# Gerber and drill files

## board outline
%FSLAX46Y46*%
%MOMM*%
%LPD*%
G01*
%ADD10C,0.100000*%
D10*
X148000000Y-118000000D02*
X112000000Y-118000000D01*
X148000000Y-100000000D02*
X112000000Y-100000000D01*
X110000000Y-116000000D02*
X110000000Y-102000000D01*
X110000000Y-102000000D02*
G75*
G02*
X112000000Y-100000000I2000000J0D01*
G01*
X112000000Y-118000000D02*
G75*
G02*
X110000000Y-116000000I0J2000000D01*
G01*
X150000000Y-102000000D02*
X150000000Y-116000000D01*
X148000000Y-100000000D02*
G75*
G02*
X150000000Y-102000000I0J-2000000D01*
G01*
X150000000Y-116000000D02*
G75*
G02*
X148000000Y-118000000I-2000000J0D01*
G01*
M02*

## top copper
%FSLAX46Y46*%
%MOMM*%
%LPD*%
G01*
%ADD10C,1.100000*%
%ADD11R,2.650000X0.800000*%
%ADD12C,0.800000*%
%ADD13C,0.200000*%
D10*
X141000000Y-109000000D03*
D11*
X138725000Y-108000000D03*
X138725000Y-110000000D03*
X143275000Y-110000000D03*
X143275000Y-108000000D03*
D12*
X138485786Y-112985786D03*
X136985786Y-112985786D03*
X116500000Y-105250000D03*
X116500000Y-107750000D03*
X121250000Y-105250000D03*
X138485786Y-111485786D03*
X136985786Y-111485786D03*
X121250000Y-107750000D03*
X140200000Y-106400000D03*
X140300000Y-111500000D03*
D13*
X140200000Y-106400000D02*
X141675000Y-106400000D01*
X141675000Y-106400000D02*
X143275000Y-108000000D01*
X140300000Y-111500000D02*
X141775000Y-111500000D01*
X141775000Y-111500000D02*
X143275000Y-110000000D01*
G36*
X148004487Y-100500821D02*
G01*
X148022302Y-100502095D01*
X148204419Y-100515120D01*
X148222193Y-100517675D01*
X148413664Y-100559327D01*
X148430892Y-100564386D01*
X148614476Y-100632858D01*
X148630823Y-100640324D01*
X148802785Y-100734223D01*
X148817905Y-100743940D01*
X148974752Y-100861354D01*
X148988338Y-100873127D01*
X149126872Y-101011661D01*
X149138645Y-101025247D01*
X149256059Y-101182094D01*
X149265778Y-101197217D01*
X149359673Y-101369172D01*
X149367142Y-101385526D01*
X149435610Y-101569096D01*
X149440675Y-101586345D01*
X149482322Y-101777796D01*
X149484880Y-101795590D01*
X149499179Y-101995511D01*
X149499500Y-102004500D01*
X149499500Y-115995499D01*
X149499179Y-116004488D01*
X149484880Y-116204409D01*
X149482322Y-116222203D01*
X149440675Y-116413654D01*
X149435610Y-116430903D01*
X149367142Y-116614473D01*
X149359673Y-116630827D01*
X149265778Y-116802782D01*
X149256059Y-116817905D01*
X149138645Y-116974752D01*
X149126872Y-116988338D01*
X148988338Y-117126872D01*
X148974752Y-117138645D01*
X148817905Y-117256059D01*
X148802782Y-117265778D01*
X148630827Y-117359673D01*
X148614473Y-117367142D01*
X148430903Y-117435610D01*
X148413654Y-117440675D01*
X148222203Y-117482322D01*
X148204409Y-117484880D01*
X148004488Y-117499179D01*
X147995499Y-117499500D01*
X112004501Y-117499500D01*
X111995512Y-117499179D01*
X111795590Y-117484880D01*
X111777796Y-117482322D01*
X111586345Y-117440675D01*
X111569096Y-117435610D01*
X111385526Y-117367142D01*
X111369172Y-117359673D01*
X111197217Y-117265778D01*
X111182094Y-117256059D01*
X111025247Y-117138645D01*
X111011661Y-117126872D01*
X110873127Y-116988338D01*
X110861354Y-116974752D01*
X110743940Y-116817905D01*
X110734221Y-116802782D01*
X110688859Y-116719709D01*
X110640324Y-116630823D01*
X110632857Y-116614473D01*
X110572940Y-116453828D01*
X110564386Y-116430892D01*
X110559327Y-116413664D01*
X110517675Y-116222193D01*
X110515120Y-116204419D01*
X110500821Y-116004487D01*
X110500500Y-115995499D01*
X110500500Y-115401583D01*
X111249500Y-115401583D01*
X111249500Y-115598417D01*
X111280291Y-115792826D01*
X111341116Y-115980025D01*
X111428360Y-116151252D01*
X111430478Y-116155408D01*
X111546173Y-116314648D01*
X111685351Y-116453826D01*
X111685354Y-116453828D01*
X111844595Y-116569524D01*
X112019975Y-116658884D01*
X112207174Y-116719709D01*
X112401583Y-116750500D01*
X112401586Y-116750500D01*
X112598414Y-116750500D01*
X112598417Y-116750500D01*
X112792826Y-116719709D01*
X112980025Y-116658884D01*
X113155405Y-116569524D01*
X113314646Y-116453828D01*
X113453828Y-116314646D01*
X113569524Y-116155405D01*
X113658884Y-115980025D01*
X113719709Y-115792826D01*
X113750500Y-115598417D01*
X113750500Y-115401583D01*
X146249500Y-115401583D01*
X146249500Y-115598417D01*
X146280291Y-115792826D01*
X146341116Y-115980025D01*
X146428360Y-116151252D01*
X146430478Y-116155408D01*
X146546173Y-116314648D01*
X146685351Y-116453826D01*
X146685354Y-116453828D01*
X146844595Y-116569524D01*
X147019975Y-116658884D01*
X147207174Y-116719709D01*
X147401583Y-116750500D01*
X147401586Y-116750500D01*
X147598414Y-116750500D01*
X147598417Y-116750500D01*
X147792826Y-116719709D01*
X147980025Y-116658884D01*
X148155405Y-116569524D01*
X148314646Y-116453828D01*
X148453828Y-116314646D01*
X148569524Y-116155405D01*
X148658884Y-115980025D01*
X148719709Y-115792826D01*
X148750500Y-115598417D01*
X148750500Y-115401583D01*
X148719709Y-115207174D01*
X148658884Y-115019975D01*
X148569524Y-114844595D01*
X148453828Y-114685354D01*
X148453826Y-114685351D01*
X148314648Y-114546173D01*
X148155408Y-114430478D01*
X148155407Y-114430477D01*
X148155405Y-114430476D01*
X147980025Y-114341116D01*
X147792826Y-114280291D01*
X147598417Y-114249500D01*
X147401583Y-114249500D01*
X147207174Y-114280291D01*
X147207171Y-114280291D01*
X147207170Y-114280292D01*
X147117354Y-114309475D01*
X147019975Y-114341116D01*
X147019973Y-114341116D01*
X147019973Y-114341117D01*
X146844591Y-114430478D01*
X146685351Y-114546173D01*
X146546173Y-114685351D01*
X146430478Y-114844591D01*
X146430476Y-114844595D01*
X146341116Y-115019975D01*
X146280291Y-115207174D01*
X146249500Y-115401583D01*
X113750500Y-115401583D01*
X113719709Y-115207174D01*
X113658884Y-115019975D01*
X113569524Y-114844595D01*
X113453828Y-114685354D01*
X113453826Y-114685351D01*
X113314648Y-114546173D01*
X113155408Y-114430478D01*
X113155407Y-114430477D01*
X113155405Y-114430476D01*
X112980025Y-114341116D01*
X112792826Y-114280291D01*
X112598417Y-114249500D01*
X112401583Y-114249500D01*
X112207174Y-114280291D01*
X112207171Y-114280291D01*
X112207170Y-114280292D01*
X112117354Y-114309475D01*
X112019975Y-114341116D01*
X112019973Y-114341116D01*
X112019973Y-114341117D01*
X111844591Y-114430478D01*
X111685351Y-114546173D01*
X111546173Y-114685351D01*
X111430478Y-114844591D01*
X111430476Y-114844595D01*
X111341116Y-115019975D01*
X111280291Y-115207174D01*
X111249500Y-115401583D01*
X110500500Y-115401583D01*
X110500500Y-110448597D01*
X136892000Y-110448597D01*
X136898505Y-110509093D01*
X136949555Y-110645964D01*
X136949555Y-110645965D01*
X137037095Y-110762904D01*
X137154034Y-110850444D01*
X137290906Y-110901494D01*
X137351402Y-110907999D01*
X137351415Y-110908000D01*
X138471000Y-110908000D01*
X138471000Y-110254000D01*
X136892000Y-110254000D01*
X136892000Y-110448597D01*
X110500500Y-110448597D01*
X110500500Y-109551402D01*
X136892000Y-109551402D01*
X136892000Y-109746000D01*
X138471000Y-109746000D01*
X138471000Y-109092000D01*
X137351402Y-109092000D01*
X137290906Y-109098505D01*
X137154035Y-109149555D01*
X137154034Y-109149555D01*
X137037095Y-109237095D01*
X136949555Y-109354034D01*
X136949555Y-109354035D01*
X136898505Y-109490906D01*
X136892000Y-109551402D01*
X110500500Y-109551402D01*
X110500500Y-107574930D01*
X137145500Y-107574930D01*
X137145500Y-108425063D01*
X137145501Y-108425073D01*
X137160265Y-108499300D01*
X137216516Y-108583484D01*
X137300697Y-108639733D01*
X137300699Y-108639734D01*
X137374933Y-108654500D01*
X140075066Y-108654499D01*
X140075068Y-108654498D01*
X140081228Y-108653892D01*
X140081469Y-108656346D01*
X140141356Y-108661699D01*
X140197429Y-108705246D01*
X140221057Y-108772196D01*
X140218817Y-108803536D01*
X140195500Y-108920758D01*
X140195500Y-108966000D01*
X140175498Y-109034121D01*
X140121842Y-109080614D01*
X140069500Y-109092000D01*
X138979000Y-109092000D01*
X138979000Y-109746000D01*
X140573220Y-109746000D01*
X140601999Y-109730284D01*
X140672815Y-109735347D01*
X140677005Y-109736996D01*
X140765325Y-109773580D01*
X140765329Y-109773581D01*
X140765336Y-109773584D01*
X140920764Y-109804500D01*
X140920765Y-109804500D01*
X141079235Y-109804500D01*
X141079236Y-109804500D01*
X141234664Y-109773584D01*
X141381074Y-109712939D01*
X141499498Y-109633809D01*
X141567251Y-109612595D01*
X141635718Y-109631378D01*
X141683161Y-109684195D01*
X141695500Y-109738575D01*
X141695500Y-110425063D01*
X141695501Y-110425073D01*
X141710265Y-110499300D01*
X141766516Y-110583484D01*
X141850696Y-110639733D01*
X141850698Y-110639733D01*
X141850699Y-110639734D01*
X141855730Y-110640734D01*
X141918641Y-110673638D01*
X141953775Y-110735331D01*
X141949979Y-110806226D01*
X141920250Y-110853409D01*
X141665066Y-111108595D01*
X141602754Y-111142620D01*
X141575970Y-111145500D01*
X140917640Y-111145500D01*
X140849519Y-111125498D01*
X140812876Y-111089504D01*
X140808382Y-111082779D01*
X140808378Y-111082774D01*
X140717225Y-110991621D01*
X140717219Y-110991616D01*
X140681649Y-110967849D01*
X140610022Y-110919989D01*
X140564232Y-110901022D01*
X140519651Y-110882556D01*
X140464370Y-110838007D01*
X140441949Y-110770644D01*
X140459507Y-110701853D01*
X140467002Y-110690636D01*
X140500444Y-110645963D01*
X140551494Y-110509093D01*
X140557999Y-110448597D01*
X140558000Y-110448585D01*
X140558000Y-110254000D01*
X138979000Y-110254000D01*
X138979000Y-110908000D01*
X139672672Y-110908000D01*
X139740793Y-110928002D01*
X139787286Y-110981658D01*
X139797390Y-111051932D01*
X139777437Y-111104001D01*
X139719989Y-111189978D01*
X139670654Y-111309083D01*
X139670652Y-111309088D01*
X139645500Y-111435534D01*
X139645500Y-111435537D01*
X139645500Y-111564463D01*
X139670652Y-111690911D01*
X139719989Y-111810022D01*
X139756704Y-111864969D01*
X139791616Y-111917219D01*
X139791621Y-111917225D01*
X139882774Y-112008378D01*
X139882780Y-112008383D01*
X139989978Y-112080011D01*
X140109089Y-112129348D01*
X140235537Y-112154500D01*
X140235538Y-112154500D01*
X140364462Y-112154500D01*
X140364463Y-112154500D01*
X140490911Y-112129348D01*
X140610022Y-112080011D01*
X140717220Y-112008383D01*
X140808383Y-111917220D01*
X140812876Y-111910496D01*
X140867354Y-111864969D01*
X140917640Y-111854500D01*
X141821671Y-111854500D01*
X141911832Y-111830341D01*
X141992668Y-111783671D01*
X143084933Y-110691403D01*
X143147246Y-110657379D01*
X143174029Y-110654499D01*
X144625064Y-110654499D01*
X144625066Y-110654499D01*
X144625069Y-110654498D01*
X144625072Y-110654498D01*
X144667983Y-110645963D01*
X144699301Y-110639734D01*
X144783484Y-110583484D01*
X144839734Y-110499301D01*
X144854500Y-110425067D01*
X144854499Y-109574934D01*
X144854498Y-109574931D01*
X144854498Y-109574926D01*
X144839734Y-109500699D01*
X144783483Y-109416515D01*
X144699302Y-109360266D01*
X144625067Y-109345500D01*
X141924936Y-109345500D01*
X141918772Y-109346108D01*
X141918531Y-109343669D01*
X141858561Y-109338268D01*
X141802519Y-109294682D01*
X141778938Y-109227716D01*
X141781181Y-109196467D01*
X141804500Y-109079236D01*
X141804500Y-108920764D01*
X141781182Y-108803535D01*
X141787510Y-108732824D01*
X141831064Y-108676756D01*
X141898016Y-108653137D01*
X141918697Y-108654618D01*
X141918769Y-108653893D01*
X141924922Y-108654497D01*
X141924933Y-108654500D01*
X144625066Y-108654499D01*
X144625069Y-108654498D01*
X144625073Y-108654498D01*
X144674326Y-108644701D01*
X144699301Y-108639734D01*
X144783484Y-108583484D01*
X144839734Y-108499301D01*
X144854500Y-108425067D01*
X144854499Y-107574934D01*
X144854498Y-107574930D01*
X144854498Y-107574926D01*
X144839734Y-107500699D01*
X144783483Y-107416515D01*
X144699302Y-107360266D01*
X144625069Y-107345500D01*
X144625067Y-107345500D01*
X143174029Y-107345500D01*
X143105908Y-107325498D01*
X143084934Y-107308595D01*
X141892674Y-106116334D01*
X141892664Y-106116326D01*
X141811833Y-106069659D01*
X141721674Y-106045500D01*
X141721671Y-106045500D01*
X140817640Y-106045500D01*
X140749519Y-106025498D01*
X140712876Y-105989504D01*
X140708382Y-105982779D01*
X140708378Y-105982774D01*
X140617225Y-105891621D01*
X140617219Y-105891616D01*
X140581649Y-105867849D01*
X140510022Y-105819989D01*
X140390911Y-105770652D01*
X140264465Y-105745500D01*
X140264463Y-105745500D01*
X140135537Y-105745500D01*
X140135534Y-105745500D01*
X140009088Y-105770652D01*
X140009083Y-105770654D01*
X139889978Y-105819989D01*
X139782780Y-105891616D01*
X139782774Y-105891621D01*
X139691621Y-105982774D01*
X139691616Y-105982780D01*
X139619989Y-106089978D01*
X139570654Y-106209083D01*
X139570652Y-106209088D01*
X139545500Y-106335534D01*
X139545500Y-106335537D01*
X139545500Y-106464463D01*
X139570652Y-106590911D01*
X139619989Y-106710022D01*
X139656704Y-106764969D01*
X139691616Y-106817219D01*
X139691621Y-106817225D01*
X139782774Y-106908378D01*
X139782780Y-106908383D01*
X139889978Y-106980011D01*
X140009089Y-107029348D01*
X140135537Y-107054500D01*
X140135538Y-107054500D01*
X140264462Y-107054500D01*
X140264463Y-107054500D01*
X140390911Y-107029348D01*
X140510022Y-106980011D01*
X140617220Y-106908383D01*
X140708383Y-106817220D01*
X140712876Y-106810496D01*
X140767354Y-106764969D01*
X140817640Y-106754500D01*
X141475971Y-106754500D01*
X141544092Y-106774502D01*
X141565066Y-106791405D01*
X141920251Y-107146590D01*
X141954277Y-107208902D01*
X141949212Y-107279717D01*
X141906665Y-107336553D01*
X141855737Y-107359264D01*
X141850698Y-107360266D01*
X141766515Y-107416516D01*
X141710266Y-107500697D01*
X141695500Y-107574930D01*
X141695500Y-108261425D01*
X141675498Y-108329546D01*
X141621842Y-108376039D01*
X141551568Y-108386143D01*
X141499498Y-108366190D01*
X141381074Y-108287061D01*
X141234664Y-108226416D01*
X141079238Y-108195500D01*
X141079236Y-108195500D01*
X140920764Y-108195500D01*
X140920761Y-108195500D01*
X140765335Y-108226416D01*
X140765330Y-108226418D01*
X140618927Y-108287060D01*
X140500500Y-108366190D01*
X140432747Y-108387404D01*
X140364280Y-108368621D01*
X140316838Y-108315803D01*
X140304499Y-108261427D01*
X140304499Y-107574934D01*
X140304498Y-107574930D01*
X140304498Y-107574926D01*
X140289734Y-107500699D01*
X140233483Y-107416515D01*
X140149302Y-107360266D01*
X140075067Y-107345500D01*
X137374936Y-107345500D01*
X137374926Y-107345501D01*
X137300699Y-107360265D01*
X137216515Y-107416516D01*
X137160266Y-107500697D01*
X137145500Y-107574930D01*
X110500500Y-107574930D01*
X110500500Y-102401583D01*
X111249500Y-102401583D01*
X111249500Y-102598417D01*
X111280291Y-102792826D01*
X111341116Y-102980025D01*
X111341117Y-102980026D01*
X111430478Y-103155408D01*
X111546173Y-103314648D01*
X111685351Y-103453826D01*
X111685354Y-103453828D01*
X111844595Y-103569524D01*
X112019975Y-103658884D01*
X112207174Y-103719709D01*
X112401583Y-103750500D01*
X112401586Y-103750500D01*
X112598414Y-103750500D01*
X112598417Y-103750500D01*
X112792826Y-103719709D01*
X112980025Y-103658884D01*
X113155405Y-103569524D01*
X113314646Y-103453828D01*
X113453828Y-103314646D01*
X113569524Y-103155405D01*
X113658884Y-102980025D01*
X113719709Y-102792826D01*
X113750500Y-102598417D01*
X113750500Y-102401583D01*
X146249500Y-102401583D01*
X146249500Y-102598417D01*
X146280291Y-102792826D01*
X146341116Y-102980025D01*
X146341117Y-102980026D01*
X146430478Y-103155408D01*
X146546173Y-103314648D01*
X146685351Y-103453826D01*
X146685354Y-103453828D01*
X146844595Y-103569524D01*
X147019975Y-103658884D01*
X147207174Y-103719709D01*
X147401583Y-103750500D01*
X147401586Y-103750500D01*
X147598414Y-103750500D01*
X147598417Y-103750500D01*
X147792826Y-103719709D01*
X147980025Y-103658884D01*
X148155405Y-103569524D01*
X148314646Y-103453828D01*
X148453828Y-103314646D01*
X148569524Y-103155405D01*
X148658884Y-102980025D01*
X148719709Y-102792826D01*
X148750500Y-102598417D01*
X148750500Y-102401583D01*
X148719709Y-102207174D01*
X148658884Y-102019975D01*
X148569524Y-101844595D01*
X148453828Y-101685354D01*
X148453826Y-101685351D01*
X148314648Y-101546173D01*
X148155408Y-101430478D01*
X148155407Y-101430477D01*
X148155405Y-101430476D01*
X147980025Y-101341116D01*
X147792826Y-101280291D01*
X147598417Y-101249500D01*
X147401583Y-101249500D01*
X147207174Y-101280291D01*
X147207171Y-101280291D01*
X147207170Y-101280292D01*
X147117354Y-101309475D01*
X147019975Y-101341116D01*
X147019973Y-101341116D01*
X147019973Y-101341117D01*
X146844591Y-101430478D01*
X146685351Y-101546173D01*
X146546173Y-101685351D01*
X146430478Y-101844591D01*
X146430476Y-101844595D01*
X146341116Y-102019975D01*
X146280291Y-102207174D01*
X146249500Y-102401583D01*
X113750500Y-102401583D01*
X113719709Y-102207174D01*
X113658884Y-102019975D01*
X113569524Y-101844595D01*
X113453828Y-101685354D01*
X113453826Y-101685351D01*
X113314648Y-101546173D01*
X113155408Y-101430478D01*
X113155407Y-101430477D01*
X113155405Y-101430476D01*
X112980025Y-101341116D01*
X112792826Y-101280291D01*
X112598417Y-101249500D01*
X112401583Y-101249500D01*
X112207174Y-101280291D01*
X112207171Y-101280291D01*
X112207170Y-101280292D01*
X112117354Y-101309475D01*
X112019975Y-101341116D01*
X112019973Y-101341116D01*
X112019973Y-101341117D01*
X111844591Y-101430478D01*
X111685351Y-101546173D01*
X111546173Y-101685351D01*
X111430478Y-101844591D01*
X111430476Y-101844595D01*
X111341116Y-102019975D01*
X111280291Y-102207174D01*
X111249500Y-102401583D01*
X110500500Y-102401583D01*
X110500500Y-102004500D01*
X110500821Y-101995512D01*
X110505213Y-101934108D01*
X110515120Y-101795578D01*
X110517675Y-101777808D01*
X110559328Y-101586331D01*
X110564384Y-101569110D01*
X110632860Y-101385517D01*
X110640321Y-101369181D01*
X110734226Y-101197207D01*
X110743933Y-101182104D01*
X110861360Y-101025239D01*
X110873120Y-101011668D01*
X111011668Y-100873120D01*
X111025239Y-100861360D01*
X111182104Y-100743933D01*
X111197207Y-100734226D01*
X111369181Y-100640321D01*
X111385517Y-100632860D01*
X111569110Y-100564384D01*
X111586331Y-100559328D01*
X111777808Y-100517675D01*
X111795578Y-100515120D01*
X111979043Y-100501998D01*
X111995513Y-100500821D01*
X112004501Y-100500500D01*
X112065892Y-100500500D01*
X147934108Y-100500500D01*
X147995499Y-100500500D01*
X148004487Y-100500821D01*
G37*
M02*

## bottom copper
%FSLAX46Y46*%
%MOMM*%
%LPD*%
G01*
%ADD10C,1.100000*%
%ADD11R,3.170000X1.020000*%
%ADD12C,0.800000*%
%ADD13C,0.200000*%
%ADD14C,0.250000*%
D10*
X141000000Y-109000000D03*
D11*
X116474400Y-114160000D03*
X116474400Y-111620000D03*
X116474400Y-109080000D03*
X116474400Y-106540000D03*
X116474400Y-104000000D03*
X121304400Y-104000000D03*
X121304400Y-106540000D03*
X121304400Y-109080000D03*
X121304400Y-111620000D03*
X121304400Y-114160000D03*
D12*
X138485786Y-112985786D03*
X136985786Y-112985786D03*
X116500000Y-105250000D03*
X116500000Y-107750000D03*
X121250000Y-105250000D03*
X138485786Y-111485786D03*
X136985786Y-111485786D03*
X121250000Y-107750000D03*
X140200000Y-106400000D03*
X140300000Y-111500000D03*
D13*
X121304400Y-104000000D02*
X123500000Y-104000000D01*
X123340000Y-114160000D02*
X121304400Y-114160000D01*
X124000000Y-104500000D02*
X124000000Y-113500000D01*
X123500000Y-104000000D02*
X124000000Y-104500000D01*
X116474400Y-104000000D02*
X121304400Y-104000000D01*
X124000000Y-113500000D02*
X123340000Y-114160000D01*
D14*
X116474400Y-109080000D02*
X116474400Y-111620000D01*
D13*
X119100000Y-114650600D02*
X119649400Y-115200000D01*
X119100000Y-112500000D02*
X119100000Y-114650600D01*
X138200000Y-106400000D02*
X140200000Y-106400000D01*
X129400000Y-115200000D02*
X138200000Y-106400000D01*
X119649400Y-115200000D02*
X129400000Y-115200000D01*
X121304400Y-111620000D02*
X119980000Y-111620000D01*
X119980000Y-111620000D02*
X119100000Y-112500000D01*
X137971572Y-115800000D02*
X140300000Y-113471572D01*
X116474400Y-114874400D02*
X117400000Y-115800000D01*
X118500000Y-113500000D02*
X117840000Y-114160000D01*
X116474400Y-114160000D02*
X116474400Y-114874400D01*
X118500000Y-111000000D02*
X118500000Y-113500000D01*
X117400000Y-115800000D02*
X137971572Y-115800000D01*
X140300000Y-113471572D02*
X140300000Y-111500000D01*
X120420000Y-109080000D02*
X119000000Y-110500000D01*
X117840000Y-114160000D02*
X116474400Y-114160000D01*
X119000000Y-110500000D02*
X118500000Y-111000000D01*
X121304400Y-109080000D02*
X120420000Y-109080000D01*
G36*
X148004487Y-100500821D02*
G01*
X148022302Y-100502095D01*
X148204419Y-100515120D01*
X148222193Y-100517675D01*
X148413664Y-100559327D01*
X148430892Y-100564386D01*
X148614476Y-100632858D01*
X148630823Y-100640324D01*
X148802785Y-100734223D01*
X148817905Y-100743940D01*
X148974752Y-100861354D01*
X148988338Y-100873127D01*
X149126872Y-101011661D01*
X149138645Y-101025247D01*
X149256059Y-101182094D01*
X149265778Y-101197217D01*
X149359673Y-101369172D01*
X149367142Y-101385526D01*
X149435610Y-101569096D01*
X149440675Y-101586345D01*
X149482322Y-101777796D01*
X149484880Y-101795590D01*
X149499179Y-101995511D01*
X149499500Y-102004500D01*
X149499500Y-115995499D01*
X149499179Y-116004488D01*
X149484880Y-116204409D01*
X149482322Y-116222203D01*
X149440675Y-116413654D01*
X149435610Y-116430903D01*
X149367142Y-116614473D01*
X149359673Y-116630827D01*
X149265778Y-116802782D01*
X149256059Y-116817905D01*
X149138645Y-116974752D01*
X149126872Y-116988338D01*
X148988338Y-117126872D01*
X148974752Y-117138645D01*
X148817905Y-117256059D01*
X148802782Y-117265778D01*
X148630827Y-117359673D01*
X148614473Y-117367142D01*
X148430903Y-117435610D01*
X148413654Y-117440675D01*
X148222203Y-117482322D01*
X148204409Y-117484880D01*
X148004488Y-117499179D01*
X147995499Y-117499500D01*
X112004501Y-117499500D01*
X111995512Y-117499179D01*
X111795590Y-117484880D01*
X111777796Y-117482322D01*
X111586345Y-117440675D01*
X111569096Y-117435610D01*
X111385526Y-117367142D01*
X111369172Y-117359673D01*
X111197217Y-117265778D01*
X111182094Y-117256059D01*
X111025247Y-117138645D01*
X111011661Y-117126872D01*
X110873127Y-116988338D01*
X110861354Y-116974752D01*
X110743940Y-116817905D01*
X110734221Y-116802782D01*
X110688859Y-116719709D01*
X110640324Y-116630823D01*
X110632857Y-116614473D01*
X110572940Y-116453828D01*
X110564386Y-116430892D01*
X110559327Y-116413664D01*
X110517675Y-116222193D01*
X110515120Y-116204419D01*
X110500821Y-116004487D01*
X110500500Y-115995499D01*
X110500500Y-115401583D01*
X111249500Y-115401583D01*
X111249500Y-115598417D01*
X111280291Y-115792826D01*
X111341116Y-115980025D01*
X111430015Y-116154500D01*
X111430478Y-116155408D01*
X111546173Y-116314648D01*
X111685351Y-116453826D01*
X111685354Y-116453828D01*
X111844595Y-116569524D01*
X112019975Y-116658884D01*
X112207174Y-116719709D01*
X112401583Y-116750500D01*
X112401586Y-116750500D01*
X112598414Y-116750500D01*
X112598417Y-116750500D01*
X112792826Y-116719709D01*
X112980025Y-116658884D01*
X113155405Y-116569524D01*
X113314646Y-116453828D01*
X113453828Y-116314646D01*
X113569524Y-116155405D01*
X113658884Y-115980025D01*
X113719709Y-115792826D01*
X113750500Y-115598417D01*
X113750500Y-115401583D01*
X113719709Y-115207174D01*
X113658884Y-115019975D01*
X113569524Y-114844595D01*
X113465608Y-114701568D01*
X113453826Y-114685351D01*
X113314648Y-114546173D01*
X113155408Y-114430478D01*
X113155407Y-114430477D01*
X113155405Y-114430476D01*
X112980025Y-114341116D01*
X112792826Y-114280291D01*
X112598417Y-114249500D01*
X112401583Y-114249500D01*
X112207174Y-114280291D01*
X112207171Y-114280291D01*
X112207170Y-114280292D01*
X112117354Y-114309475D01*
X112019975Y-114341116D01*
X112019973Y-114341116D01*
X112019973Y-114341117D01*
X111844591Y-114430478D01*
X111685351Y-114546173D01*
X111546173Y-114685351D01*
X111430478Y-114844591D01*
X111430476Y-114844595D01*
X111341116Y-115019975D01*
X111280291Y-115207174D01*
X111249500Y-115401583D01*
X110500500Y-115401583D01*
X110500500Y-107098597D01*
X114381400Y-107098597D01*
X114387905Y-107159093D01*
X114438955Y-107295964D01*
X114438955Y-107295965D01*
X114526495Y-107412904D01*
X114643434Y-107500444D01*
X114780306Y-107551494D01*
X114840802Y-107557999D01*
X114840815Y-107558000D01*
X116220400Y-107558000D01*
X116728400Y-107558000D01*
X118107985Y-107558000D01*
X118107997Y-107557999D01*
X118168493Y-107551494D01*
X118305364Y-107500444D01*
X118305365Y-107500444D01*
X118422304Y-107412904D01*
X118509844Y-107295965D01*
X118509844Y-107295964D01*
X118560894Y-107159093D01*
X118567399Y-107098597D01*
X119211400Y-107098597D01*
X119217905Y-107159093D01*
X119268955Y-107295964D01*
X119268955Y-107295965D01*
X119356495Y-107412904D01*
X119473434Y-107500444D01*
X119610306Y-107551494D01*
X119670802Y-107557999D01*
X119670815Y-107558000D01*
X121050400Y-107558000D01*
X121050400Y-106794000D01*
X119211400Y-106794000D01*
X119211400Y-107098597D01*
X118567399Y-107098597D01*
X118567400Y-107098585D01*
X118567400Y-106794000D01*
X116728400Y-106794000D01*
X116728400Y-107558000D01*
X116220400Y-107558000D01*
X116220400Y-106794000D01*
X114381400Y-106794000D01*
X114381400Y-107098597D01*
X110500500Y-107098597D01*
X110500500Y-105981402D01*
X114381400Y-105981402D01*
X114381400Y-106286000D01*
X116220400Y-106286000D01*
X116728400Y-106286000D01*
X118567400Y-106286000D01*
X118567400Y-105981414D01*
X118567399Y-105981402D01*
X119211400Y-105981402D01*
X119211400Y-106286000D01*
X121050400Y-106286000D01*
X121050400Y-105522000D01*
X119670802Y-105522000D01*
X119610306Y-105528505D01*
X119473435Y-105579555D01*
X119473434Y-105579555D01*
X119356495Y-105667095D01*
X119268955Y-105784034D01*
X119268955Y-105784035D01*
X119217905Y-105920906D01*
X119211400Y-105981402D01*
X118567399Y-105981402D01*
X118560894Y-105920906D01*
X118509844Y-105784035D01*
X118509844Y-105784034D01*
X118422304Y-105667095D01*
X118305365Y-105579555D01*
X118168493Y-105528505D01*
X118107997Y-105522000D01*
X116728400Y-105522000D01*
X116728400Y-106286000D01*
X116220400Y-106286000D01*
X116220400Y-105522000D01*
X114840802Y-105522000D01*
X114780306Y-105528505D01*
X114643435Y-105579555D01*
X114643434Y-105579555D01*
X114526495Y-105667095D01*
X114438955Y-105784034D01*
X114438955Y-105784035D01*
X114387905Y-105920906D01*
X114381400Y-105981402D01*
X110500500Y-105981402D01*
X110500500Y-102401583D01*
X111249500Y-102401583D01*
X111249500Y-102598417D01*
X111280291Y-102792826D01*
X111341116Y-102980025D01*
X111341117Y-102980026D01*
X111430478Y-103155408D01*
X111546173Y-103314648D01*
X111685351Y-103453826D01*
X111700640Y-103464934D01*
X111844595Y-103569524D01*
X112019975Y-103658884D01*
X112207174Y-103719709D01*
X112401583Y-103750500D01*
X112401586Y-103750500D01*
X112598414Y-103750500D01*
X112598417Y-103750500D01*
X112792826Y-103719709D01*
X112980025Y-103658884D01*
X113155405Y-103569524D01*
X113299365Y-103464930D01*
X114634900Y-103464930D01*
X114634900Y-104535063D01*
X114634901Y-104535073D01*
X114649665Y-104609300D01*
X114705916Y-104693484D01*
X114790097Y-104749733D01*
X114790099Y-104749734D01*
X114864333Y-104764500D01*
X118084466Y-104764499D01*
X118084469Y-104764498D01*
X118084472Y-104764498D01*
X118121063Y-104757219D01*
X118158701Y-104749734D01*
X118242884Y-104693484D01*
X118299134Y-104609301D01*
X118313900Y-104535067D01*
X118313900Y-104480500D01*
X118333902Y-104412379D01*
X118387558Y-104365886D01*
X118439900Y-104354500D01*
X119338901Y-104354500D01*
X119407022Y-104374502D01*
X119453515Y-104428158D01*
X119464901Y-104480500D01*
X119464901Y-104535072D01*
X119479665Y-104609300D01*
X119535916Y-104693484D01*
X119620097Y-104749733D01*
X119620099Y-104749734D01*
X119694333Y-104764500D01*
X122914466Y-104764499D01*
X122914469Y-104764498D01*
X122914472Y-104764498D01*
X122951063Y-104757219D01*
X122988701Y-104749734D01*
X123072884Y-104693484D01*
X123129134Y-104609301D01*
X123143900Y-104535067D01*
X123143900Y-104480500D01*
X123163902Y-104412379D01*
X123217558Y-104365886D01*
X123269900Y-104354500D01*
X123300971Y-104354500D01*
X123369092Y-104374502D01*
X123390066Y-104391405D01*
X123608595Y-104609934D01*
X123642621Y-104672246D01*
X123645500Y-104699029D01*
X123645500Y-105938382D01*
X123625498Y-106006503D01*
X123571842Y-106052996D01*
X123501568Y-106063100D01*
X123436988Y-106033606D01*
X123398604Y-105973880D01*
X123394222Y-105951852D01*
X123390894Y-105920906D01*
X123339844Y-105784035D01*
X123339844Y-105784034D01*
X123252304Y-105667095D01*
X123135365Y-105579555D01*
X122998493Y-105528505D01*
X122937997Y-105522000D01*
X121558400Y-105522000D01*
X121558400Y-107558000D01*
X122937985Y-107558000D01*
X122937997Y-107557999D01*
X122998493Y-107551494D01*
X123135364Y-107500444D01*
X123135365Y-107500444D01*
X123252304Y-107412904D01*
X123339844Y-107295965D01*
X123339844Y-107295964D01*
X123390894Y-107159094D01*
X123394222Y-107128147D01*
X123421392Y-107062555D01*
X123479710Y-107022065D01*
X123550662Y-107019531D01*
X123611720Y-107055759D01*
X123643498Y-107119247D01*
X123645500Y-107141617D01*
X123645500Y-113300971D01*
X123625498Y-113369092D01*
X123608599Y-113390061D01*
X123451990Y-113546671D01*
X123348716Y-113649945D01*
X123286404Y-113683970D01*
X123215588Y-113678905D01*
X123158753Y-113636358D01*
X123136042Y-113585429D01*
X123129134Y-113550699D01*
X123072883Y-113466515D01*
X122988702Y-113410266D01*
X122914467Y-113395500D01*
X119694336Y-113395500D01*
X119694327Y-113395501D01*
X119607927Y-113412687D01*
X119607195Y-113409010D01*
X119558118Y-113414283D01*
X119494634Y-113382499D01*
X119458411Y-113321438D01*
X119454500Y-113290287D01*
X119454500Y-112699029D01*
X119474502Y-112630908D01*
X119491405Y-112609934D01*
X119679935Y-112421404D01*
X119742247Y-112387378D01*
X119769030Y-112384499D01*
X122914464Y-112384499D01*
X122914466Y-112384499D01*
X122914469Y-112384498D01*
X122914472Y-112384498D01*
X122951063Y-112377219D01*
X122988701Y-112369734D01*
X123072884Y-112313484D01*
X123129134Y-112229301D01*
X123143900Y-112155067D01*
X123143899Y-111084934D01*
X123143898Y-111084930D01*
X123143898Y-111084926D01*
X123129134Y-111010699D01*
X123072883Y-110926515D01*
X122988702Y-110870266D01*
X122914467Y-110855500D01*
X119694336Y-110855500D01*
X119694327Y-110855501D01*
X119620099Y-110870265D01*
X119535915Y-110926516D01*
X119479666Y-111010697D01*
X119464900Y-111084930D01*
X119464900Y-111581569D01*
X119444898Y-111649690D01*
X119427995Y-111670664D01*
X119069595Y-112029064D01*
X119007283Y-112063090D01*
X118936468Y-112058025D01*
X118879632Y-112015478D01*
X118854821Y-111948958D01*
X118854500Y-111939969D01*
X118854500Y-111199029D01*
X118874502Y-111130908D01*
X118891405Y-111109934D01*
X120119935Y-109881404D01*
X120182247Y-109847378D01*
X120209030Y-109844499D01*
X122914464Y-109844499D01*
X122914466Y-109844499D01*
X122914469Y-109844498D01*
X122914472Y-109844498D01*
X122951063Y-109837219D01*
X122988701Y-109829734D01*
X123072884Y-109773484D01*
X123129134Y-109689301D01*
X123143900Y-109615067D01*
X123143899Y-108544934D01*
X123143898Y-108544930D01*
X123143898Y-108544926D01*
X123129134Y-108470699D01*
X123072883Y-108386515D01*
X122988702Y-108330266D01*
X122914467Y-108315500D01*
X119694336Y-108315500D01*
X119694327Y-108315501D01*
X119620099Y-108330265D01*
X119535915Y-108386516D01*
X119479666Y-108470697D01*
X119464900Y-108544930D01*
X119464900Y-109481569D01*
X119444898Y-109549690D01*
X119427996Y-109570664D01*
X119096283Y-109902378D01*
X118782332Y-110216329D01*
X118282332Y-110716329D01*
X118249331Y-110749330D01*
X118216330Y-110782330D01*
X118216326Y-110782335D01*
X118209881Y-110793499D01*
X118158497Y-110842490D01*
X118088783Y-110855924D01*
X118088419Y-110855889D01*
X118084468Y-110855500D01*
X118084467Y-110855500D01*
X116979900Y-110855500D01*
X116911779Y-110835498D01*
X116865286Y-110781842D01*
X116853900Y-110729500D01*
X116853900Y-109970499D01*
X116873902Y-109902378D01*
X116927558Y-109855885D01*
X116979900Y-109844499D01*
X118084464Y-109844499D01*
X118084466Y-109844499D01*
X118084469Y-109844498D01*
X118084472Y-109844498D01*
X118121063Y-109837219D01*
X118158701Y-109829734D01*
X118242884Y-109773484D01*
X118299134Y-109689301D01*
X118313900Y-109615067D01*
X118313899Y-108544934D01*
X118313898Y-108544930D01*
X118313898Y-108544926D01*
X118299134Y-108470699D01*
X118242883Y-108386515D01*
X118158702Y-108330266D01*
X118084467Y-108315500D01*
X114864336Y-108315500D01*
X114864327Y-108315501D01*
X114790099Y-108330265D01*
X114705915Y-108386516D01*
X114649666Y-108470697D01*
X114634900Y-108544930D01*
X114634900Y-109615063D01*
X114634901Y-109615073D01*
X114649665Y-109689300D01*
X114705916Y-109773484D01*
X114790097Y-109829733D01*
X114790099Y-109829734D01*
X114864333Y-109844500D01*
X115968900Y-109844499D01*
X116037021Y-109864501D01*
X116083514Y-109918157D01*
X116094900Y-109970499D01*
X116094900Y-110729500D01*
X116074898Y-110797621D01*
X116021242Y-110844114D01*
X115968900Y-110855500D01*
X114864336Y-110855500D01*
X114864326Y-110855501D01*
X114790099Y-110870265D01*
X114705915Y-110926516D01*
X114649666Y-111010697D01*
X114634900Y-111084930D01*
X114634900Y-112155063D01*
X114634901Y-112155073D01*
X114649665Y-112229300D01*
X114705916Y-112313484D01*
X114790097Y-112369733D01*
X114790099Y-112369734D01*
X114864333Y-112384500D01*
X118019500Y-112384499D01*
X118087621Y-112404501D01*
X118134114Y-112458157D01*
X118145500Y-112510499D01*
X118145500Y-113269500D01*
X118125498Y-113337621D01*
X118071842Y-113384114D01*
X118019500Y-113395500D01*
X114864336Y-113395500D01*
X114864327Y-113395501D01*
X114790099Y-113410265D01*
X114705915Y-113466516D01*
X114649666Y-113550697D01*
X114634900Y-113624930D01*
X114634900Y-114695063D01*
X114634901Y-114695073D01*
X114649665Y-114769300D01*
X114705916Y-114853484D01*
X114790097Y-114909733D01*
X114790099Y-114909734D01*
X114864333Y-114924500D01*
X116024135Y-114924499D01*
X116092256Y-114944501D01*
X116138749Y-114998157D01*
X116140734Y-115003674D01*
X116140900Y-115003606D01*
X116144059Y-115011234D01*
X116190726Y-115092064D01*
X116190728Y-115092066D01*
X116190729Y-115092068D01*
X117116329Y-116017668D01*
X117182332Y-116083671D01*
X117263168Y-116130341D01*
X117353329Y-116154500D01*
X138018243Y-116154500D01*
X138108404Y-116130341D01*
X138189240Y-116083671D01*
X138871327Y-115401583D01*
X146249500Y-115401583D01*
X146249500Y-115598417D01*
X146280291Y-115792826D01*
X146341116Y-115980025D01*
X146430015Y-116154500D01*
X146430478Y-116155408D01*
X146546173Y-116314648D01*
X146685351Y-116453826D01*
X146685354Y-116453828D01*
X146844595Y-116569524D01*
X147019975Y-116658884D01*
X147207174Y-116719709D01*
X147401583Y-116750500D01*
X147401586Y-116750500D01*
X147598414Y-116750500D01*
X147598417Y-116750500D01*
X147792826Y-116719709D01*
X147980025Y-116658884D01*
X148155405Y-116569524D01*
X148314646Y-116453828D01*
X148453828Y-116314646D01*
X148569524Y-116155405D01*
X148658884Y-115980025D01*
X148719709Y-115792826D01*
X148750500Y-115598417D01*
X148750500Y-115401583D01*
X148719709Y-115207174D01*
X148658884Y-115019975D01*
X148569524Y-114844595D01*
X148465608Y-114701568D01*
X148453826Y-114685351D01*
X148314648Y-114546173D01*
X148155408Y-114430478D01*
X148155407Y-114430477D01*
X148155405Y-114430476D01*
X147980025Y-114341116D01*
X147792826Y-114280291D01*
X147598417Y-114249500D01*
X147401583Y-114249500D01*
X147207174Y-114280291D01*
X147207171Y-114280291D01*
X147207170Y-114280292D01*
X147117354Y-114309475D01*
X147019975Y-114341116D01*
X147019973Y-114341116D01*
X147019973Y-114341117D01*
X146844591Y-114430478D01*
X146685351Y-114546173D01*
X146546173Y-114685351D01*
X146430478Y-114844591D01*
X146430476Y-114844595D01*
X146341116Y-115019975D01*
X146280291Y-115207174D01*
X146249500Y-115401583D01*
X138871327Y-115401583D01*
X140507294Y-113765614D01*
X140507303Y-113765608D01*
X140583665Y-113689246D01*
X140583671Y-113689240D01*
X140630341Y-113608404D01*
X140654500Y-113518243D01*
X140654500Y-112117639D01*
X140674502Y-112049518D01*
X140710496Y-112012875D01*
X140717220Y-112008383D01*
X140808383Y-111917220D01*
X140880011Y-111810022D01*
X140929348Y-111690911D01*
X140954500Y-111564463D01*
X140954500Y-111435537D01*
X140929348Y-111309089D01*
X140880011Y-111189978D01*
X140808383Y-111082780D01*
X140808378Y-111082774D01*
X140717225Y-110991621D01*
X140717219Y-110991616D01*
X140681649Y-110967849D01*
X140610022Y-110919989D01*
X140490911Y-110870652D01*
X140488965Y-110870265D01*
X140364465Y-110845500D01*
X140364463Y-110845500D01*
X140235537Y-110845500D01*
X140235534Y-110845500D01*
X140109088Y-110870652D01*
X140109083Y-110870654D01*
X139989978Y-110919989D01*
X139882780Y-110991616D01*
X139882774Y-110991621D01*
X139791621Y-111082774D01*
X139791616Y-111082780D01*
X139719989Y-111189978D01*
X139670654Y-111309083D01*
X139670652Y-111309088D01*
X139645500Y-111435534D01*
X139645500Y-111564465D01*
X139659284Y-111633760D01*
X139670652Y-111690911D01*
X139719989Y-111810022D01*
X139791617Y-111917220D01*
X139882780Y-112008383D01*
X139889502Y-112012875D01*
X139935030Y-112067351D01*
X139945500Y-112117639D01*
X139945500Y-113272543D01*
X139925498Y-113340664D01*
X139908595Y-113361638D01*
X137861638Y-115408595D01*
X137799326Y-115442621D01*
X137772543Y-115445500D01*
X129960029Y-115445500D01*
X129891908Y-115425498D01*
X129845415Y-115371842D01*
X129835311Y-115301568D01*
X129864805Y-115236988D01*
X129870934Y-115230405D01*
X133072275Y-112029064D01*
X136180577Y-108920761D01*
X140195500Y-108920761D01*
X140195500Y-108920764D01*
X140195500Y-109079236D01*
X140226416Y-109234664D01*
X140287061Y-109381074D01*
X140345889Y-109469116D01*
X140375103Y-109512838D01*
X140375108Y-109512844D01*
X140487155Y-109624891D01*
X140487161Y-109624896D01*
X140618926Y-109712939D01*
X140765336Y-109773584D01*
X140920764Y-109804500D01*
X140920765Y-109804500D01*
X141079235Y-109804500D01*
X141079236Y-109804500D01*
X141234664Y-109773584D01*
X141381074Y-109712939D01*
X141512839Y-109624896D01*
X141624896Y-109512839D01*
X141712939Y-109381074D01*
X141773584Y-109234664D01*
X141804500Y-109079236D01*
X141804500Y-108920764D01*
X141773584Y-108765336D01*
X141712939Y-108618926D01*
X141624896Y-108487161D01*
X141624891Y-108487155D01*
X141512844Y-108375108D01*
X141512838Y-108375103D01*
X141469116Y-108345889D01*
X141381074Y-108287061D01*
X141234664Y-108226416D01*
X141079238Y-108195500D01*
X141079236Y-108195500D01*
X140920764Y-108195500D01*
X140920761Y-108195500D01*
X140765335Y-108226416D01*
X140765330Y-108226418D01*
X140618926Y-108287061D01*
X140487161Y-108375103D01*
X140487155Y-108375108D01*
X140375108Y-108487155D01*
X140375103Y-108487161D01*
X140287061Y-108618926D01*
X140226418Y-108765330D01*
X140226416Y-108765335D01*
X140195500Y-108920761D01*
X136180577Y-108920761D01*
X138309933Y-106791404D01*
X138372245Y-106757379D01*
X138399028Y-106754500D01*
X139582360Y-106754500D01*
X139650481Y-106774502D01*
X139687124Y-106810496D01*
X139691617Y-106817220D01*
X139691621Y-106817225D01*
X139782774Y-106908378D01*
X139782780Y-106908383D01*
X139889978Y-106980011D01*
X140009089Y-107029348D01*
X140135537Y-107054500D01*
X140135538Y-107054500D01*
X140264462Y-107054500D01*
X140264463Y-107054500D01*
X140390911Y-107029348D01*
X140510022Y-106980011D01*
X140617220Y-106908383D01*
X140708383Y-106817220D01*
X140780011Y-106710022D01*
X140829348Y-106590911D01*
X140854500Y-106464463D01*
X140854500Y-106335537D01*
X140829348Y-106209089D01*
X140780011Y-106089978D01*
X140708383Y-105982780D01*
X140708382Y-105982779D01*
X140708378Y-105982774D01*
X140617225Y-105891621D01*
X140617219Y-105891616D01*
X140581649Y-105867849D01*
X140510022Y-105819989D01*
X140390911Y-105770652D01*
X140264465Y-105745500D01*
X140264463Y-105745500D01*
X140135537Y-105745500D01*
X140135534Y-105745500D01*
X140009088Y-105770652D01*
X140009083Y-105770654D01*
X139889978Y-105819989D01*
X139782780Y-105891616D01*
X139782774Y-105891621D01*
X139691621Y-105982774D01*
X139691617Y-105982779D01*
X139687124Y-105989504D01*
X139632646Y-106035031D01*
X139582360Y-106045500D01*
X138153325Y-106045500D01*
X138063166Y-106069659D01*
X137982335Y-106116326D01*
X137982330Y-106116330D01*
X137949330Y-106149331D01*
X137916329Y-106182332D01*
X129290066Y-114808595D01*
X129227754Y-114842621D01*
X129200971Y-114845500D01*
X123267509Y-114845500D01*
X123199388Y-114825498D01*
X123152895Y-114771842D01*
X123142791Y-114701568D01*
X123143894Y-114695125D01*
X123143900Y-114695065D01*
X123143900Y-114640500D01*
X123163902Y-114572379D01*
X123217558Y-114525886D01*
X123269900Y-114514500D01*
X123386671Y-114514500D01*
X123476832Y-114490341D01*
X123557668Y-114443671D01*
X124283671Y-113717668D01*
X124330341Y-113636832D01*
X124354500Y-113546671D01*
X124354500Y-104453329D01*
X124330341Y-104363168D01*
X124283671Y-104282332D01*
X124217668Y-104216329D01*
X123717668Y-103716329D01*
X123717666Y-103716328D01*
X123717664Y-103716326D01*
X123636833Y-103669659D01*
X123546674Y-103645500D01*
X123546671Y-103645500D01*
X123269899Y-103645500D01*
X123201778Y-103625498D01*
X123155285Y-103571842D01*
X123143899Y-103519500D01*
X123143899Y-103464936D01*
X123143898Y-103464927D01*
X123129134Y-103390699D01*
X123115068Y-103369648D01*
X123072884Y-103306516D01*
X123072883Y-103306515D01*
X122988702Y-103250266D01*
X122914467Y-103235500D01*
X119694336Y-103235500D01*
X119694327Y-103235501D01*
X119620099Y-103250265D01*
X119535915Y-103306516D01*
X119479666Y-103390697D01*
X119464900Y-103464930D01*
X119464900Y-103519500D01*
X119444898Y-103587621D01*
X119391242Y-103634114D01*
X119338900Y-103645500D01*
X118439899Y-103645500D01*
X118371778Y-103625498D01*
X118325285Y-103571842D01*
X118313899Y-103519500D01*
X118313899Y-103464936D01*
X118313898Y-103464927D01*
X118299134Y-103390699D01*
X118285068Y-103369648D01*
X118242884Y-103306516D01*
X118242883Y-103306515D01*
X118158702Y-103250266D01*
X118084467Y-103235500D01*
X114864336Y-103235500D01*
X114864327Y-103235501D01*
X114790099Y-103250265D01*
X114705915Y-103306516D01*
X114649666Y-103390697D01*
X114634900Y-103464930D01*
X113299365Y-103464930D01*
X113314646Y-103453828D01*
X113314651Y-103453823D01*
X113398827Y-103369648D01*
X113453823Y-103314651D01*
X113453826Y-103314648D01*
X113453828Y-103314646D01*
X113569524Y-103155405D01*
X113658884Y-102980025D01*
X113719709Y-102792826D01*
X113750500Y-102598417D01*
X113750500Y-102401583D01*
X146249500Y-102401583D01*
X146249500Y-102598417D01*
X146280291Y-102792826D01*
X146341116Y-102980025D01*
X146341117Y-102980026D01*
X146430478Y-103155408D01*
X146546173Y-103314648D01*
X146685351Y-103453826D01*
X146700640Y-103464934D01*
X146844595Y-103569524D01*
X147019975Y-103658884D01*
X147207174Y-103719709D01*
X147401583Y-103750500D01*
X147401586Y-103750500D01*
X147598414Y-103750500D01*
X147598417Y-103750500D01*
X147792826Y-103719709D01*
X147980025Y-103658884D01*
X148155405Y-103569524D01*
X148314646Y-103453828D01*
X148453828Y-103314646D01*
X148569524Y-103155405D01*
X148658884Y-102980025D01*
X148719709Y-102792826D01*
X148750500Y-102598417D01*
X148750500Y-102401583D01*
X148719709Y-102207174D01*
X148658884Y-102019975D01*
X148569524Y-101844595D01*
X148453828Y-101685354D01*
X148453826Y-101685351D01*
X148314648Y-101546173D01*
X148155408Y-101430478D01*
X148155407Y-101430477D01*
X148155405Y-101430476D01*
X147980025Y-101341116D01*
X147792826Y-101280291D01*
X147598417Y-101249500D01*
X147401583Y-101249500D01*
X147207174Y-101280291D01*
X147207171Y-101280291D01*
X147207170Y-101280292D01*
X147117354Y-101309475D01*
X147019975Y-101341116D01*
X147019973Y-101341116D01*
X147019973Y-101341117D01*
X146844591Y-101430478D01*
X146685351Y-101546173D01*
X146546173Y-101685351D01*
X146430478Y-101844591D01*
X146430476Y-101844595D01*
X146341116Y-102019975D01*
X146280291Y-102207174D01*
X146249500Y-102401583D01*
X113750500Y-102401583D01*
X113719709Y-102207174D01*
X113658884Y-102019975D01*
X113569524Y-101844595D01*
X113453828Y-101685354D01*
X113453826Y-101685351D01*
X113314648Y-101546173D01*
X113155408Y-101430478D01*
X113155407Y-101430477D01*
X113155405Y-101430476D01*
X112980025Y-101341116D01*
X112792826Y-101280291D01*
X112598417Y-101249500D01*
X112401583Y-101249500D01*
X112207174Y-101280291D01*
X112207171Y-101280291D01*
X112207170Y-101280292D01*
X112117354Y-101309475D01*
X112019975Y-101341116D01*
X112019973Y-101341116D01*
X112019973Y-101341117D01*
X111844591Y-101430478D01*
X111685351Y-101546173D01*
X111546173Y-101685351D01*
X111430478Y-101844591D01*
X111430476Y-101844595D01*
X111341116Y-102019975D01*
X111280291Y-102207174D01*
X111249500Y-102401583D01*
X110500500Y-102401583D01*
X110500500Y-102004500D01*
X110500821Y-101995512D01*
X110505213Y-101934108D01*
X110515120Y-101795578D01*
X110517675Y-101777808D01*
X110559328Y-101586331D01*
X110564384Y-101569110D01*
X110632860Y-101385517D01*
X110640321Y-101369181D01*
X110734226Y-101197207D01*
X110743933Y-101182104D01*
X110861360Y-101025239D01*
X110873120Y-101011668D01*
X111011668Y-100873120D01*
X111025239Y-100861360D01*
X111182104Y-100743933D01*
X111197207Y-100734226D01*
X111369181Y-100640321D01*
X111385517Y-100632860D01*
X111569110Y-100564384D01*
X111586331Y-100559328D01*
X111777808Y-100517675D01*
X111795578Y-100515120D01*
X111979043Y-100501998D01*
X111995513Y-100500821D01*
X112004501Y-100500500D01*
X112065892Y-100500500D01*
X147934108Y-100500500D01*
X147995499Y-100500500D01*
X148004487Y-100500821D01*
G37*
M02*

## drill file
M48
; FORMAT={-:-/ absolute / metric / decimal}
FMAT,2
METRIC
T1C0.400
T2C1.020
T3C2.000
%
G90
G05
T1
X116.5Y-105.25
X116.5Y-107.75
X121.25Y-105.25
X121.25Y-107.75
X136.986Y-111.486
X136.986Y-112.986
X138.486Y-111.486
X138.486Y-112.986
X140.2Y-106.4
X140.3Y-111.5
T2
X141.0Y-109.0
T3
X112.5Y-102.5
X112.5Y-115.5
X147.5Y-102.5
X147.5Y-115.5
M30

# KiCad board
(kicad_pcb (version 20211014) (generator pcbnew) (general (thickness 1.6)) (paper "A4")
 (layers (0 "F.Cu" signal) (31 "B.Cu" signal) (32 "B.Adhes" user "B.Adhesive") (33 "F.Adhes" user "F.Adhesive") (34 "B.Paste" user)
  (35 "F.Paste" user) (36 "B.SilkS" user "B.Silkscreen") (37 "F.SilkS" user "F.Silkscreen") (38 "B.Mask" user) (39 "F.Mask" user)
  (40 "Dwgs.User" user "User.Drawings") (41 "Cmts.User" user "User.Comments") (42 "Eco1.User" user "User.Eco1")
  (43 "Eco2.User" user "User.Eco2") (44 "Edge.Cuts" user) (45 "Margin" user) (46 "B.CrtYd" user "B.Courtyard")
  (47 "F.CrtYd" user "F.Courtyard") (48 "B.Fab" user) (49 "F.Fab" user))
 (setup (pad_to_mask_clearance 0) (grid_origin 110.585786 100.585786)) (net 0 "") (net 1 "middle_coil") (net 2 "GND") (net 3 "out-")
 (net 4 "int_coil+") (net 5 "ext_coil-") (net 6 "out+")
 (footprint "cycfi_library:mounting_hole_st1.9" (layer "F.Cu") (at 147.5 115.5 180)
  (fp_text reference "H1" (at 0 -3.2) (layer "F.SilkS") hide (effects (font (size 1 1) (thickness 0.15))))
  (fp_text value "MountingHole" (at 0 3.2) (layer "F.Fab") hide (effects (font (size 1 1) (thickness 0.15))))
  (pad "" np_thru_hole circle locked (at 0 0 180) (size 2 2) (drill 2) (layers *.Cu *.Mask)))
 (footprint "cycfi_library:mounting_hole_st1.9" (layer "F.Cu") (at 147.5 102.5 180)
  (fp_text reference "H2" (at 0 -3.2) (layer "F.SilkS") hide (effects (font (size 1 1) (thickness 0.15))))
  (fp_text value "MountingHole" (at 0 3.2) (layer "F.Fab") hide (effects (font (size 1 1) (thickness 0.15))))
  (pad "" np_thru_hole circle locked (at 0 0 180) (size 2 2) (drill 2) (layers *.Cu *.Mask)))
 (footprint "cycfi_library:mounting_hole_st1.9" (layer "F.Cu") (at 112.5 115.5 180)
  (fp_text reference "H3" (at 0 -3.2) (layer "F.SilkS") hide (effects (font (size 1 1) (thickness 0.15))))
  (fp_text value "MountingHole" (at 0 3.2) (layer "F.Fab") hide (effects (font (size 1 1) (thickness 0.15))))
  (pad "" np_thru_hole circle locked (at 0 0 180) (size 2 2) (drill 2) (layers *.Cu *.Mask)))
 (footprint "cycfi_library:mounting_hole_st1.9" (layer "F.Cu") (at 112.5 102.5 180)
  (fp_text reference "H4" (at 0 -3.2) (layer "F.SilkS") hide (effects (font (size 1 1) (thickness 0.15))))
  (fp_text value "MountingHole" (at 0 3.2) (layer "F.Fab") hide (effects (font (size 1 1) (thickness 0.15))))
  (pad "" np_thru_hole circle locked (at 0 0 180) (size 2 2) (drill 2) (layers *.Cu *.Mask)))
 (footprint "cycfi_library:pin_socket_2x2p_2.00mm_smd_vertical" (layer "F.Cu") (at 141 109)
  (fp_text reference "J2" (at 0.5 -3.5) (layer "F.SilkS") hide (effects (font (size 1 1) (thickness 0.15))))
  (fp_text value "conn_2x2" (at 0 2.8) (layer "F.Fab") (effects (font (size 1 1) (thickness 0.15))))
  (pad "" np_thru_hole circle (at 0 0) (size 1.1 1.1) (drill 1.02) (layers F&B.Cu *.Mask))
  (pad "1" smd rect (at -2.275 -1) (size 2.65 0.8) (layers "F.Cu" "F.Paste" "F.Mask") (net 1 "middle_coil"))
  (pad "2" smd rect (at -2.275 1) (size 2.65 0.8) (layers "F.Cu" "F.Paste" "F.Mask") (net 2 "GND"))
  (pad "3" smd rect (at 2.275 1) (size 2.65 0.8) (layers "F.Cu" "F.Paste" "F.Mask") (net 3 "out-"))
  (pad "4" smd rect (at 2.275 -1) (size 2.65 0.8) (layers "F.Cu" "F.Paste" "F.Mask") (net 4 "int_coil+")))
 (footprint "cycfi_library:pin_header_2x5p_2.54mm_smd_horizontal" (layer "B.Cu") (at 118.9 109.08)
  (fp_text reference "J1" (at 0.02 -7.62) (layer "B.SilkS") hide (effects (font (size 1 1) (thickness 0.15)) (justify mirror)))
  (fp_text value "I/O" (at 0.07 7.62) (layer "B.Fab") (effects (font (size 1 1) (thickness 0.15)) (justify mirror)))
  (pad "1" smd rect (at -2.4256 5.08) (size 3.17 1.02) (layers "B.Cu" "B.Paste" "B.Mask") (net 3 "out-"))
  (pad "2" smd rect (at -2.4256 2.54) (size 3.17 1.02) (layers "B.Cu" "B.Paste" "B.Mask") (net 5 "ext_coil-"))
  (pad "3" smd rect (at -2.4256 0) (size 3.17 1.02) (layers "B.Cu" "B.Paste" "B.Mask") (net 5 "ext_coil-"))
  (pad "4" smd rect (at -2.4256 -2.54) (size 3.17 1.02) (layers "B.Cu" "B.Paste" "B.Mask") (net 2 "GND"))
  (pad "5" smd rect (at -2.4256 -5.08) (size 3.17 1.02) (layers "B.Cu" "B.Paste" "B.Mask") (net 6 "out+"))
  (pad "6" smd rect (at 2.4044 -5.08) (size 3.17 1.02) (layers "B.Cu" "B.Paste" "B.Mask") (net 6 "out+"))
  (pad "7" smd rect (at 2.4044 -2.54) (size 3.17 1.02) (layers "B.Cu" "B.Paste" "B.Mask") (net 2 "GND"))
  (pad "8" smd rect (at 2.4044 0) (size 3.17 1.02) (layers "B.Cu" "B.Paste" "B.Mask") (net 3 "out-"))
  (pad "9" smd rect (at 2.4044 2.54) (size 3.17 1.02) (layers "B.Cu" "B.Paste" "B.Mask") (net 4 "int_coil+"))
  (pad "10" smd rect (at 2.4044 5.08) (size 3.17 1.02) (layers "B.Cu" "B.Paste" "B.Mask") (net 6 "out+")))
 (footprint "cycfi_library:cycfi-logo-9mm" (layer "B.Cu") (at 146.385786 108.985786 -90)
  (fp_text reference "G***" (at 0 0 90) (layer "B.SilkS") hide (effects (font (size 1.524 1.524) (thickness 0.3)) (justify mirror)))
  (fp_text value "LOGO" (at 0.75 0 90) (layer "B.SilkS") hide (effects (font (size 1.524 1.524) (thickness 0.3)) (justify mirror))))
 (gr_line (start 148 118) (end 112 118) (layer "Edge.Cuts") (width 0.1))
 (gr_line (start 148 100) (end 112 100) (layer "Edge.Cuts") (width 0.1))
 (gr_line (start 110 116) (end 110 102) (layer "Edge.Cuts") (width 0.1))
 (gr_arc (start 110 102) (mid 110.585786 100.585786) (end 112 100) (layer "Edge.Cuts") (width 0.1))
 (gr_arc (start 112 118) (mid 110.585786 117.414214) (end 110 116) (layer "Edge.Cuts") (width 0.1))
 (gr_line (start 150 102) (end 150 116) (layer "Edge.Cuts") (width 0.1))
 (gr_arc (start 148 100) (mid 149.414214 100.585786) (end 150 102) (layer "Edge.Cuts") (width 0.1))
 (gr_arc (start 150 116) (mid 149.414214 117.414214) (end 148 118) (layer "Edge.Cuts") (width 0.1))
 (via (at 138.485786 112.985786) (size 0.8) (drill 0.4) (layers "F.Cu" "B.Cu") (free) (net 2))
 (via (at 136.985786 112.985786) (size 0.8) (drill 0.4) (layers "F.Cu" "B.Cu") (free) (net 2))
 (via (at 116.5 105.25) (size 0.8) (drill 0.4) (layers "F.Cu" "B.Cu") (free) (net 2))
 (via (at 116.5 107.75) (size 0.8) (drill 0.4) (layers "F.Cu" "B.Cu") (free) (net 2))
 (via (at 121.25 105.25) (size 0.8) (drill 0.4) (layers "F.Cu" "B.Cu") (free) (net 2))
 (via (at 138.485786 111.485786) (size 0.8) (drill 0.4) (layers "F.Cu" "B.Cu") (free) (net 2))
 (via (at 136.985786 111.485786) (size 0.8) (drill 0.4) (layers "F.Cu" "B.Cu") (free) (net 2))
 (via (at 121.25 107.75) (size 0.8) (drill 0.4) (layers "F.Cu" "B.Cu") (free) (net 2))
 (segment (start 121.3044 104) (end 123.5 104) (width 0.2) (layer "B.Cu") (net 6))
 (segment (start 123.34 114.16) (end 121.3044 114.16) (width 0.2) (layer "B.Cu") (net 6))
 (segment (start 124 104.5) (end 124 113.5) (width 0.2) (layer "B.Cu") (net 6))
 (segment (start 123.5 104) (end 124 104.5) (width 0.2) (layer "B.Cu") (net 6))
 (segment (start 116.4744 104) (end 121.3044 104) (width 0.2) (layer "B.Cu") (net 6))
 (segment (start 124 113.5) (end 123.34 114.16) (width 0.2) (layer "B.Cu") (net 6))
 (segment (start 116.4744 109.08) (end 116.4744 111.62) (width 0.25) (layer "B.Cu") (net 5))
 (segment (start 140.2 106.4) (end 141.675 106.4) (width 0.2) (layer "F.Cu") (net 4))
 (segment (start 141.675 106.4) (end 143.275 108) (width 0.2) (layer "F.Cu") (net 4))
 (via (at 140.2 106.4) (size 0.8) (drill 0.4) (layers "F.Cu" "B.Cu") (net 4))
 (segment (start 119.1 114.6506) (end 119.6494 115.2) (width 0.2) (layer "B.Cu") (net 4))
 (segment (start 119.1 112.5) (end 119.1 114.6506) (width 0.2) (layer "B.Cu") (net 4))
 (segment (start 138.2 106.4) (end 140.2 106.4) (width 0.2) (layer "B.Cu") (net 4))
 (segment (start 129.4 115.2) (end 138.2 106.4) (width 0.2) (layer "B.Cu") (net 4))
 (segment (start 119.6494 115.2) (end 129.4 115.2) (width 0.2) (layer "B.Cu") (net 4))
 (segment (start 121.3044 111.62) (end 119.98 111.62) (width 0.2) (layer "B.Cu") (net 4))
 (segment (start 119.98 111.62) (end 119.1 112.5) (width 0.2) (layer "B.Cu") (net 4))
 (segment (start 140.3 111.5) (end 141.775 111.5) (width 0.2) (layer "F.Cu") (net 3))
 (segment (start 141.775 111.5) (end 143.275 110) (width 0.2) (layer "F.Cu") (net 3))
 (via (at 140.3 111.5) (size 0.8) (drill 0.4) (layers "F.Cu" "B.Cu") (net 3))
 (segment (start 137.971572 115.8) (end 140.3 113.471572) (width 0.2) (layer "B.Cu") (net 3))
 (segment (start 116.4744 114.8744) (end 117.4 115.8) (width 0.2) (layer "B.Cu") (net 3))
 (segment (start 118.5 113.5) (end 117.84 114.16) (width 0.2) (layer "B.Cu") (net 3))
 (segment (start 116.4744 114.16) (end 116.4744 114.8744) (width 0.2) (layer "B.Cu") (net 3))
 (segment (start 118.5 111) (end 118.5 113.5) (width 0.2) (layer "B.Cu") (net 3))
 (segment (start 117.4 115.8) (end 137.971572 115.8) (width 0.2) (layer "B.Cu") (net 3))
 (segment (start 140.3 113.471572) (end 140.3 111.5) (width 0.2) (layer "B.Cu") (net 3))
 (segment (start 120.42 109.08) (end 119 110.5) (width 0.2) (layer "B.Cu") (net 3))
 (segment (start 117.84 114.16) (end 116.4744 114.16) (width 0.2) (layer "B.Cu") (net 3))
 (segment (start 119 110.5) (end 118.5 111) (width 0.2) (layer "B.Cu") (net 3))
 (segment (start 121.3044 109.08) (end 120.42 109.08) (width 0.2) (layer "B.Cu") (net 3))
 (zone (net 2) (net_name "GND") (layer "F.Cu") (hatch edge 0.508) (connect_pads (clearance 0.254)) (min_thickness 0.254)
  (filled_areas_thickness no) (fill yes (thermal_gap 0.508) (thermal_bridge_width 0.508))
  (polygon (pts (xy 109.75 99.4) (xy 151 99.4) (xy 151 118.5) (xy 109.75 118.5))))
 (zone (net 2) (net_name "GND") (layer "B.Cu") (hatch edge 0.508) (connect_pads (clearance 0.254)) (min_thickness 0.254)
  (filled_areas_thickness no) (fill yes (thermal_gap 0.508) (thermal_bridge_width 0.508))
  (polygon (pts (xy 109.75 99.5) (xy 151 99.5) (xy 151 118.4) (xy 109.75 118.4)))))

